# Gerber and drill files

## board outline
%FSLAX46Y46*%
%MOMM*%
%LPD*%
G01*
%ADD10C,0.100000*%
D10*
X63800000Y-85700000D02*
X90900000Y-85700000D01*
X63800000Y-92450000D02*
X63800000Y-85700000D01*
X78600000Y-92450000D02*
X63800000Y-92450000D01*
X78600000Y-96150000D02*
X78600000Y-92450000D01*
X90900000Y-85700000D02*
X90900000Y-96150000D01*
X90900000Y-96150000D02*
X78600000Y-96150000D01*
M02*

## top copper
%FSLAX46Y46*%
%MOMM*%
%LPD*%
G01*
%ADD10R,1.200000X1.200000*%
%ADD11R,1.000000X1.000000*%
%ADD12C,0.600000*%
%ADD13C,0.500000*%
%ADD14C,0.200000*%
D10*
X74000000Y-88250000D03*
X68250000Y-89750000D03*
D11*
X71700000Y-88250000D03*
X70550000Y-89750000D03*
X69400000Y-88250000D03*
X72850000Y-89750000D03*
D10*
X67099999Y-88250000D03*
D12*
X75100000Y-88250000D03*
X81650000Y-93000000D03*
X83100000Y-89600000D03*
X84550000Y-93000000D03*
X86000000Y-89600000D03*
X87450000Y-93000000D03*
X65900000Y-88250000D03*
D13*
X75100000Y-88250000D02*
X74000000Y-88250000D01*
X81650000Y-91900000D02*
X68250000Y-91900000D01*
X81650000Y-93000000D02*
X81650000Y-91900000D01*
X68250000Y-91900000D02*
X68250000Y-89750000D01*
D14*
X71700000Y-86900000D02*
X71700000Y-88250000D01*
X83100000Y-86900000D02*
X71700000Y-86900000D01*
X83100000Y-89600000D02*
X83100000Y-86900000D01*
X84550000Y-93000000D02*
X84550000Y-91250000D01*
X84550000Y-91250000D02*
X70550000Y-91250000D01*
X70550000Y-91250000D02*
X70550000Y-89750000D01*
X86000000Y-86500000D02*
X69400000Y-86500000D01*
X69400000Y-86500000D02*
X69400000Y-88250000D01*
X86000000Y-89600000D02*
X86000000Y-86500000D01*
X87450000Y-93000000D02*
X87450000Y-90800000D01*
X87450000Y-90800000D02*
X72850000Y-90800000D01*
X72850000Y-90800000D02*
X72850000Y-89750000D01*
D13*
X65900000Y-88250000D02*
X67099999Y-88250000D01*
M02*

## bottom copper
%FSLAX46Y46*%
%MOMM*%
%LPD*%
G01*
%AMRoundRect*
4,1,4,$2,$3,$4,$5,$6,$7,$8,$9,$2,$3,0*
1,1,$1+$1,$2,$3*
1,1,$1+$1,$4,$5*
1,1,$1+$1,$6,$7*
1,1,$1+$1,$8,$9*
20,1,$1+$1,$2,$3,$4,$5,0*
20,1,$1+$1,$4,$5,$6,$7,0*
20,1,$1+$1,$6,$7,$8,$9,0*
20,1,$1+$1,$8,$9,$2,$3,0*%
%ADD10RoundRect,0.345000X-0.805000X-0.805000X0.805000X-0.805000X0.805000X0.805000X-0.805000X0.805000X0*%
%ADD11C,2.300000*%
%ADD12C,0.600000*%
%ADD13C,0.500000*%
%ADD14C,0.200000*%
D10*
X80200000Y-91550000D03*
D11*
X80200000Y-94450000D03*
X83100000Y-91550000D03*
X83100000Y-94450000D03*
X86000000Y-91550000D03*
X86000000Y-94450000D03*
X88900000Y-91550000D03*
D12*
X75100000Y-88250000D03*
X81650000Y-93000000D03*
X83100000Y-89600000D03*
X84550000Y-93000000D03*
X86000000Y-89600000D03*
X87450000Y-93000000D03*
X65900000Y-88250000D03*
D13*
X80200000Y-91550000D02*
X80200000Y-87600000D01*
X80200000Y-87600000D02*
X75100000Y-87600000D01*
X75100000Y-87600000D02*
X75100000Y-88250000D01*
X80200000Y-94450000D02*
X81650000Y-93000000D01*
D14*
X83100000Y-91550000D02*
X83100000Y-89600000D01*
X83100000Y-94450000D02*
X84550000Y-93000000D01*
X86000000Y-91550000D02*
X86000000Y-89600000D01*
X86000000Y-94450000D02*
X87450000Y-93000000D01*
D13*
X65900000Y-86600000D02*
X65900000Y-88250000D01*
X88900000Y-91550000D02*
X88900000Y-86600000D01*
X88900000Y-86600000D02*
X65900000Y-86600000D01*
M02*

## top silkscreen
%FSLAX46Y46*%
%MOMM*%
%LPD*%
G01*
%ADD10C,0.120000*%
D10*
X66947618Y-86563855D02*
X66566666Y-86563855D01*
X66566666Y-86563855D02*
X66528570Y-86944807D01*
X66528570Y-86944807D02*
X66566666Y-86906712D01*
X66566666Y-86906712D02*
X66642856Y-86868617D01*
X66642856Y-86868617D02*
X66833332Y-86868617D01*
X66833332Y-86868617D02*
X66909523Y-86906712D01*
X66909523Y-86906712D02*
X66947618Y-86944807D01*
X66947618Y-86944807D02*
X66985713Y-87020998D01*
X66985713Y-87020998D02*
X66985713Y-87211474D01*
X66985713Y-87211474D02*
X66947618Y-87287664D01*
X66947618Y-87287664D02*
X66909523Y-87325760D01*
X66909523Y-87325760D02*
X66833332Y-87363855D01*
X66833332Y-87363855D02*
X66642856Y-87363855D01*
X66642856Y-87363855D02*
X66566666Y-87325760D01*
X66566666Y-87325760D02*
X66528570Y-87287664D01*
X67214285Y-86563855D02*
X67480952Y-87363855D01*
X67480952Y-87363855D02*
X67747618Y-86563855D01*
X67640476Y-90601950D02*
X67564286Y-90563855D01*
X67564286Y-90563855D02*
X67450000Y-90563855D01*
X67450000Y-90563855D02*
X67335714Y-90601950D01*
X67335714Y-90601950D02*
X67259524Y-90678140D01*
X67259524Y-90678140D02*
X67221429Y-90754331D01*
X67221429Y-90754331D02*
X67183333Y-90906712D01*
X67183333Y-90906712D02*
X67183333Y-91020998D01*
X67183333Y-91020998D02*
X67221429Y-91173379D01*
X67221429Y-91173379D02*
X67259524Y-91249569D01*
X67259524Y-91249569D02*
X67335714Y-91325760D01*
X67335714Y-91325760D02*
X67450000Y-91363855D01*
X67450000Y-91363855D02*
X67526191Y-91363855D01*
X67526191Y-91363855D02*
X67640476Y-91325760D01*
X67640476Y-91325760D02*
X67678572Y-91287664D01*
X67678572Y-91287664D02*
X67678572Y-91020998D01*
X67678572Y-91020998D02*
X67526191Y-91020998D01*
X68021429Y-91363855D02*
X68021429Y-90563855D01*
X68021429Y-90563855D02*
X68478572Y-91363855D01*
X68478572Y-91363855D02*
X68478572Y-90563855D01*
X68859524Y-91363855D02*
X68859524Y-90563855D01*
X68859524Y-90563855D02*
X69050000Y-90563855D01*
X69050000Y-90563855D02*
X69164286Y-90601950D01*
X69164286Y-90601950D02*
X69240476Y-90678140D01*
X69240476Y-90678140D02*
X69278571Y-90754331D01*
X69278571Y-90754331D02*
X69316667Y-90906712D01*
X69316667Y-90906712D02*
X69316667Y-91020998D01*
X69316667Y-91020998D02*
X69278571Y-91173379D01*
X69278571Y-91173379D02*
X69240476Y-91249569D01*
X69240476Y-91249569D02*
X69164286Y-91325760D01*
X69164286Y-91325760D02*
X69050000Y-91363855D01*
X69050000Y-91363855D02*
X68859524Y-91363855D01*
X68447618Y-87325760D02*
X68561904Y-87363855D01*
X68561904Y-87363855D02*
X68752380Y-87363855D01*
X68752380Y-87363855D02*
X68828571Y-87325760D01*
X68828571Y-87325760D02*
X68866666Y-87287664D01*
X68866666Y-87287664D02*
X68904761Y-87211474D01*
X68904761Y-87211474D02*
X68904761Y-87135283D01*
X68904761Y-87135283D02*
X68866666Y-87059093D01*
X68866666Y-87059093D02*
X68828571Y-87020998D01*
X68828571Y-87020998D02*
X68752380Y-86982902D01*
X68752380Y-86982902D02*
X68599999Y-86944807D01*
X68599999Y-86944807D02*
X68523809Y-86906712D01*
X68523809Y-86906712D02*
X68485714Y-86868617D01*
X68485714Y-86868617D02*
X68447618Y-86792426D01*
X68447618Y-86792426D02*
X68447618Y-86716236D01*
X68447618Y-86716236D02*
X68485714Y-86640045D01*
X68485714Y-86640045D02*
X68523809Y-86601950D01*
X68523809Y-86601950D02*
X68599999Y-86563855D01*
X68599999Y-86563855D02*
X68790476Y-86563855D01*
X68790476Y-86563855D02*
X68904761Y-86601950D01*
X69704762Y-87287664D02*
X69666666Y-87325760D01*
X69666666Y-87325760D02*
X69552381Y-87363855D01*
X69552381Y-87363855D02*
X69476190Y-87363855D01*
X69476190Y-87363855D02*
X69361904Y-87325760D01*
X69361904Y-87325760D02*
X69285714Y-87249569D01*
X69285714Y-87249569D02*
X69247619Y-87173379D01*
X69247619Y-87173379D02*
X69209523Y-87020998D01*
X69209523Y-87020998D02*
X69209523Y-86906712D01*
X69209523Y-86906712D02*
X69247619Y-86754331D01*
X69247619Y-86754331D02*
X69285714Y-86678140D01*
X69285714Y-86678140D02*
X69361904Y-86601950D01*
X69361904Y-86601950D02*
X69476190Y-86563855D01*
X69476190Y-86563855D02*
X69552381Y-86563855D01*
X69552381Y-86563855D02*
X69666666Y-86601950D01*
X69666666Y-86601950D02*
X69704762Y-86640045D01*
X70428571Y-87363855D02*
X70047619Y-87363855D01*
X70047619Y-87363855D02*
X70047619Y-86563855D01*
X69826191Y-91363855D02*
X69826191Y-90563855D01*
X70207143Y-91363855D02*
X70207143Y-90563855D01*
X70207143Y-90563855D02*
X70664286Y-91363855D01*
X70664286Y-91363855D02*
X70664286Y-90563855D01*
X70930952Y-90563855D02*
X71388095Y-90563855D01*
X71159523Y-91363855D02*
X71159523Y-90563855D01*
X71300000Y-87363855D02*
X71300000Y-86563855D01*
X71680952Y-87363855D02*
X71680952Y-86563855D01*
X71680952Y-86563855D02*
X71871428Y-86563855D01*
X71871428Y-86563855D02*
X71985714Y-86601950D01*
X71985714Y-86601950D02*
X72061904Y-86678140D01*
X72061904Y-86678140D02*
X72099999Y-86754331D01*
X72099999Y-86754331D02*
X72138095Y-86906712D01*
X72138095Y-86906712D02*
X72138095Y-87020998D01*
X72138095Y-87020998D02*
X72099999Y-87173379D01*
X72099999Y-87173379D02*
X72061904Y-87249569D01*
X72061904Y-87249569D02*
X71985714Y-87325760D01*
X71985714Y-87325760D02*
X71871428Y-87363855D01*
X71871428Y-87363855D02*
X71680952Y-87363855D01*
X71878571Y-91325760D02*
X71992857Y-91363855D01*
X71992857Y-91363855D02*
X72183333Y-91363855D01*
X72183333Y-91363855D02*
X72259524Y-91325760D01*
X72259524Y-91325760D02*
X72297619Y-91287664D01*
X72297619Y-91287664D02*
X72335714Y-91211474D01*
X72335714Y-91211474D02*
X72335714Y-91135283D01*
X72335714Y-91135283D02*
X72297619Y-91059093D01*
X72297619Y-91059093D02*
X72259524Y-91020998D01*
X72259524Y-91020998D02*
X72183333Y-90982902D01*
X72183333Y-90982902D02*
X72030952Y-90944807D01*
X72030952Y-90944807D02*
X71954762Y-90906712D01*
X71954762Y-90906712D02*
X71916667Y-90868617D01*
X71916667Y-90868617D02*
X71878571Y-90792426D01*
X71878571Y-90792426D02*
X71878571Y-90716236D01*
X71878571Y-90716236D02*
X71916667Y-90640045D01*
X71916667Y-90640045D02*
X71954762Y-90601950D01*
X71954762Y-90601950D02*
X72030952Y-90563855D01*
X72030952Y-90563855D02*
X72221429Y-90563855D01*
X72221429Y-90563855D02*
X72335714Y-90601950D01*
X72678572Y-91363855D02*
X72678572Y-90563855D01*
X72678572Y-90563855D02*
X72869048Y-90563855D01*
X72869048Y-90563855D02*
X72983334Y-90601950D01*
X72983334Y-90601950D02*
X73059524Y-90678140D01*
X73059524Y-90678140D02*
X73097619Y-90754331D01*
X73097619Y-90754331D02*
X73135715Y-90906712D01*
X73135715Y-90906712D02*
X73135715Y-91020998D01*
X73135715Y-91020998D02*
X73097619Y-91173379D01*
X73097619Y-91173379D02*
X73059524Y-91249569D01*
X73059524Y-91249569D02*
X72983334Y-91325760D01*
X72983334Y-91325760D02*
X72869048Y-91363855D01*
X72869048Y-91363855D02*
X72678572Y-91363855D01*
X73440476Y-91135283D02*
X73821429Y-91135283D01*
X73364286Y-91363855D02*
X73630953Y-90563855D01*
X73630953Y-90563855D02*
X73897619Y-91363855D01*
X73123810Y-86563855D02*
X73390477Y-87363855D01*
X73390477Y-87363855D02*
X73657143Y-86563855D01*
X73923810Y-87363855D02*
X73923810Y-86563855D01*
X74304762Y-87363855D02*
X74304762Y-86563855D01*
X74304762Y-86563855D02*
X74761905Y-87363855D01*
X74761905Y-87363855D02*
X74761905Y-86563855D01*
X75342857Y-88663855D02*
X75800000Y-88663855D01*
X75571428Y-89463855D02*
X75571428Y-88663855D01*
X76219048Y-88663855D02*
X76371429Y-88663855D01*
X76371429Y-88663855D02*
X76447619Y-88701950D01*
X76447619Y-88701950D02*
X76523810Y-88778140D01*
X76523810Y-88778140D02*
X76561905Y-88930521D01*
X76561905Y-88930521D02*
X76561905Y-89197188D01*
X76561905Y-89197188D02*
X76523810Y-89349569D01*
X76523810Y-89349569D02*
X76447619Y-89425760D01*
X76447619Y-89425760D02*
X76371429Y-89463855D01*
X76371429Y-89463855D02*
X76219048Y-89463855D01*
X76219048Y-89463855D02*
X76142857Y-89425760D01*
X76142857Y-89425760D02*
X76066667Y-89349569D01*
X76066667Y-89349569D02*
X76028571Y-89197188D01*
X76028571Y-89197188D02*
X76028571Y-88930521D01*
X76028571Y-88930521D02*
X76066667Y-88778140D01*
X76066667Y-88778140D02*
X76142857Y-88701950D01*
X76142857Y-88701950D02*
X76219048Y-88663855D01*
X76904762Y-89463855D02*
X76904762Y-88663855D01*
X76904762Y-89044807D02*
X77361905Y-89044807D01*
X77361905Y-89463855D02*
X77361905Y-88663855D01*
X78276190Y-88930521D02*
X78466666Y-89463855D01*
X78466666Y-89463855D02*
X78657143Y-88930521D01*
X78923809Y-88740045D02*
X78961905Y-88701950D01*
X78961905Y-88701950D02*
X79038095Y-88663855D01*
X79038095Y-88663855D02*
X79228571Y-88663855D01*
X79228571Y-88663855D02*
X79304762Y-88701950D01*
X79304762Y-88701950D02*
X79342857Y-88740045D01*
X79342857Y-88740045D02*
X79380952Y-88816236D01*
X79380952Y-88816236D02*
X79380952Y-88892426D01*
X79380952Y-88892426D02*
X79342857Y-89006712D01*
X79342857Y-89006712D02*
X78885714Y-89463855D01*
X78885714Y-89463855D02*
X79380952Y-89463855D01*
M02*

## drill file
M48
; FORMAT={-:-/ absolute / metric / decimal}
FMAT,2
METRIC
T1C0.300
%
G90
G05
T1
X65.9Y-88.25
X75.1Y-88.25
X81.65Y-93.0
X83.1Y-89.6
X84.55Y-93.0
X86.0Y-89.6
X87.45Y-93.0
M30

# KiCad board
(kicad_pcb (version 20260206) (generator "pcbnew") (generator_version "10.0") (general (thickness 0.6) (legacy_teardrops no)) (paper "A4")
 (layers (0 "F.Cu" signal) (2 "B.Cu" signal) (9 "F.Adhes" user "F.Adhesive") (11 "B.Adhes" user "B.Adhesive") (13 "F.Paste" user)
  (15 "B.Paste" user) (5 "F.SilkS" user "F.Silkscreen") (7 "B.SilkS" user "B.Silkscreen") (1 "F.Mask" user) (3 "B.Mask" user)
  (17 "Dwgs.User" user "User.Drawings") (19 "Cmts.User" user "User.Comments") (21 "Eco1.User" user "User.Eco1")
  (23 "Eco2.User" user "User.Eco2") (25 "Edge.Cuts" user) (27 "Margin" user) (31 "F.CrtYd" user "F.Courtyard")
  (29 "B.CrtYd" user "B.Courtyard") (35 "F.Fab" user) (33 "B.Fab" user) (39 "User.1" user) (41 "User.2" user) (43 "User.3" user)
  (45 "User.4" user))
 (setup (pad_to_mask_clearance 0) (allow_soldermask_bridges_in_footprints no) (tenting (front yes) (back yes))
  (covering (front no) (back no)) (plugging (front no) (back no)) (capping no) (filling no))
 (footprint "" (layer "F.Cu") (at 70.55 89)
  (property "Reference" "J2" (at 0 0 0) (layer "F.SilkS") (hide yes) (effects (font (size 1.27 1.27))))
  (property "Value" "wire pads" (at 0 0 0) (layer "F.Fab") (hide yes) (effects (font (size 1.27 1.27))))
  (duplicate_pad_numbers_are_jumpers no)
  (pad "1" smd rect (at 3.45 -0.75) (size 1.2 1.2) (layers "F.Cu" "F.Mask") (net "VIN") (thermal_bridge_angle 45))
  (pad "2" smd rect (at -2.3 0.75) (size 1.2 1.2) (layers "F.Cu" "F.Mask") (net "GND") (thermal_bridge_angle 45))
  (pad "3" smd rect (at 1.15 -0.75) (size 1 1) (layers "F.Cu" "F.Mask") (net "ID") (thermal_bridge_angle 45))
  (pad "4" smd rect (at 0 0.75) (size 1 1) (layers "F.Cu" "F.Mask") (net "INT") (thermal_bridge_angle 45))
  (pad "5" smd rect (at -1.15 -0.75) (size 1 1) (layers "F.Cu" "F.Mask") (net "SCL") (thermal_bridge_angle 45))
  (pad "6" smd rect (at 2.3 0.75) (size 1 1) (layers "F.Cu" "F.Mask") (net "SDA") (thermal_bridge_angle 45))
  (pad "7" smd rect (at -3.450001 -0.75) (size 1.2 1.2) (layers "F.Cu" "F.Mask") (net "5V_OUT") (thermal_bridge_angle 45)))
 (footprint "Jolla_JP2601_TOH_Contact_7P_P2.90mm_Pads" (layer "F.Cu") (at 80.2 91.55)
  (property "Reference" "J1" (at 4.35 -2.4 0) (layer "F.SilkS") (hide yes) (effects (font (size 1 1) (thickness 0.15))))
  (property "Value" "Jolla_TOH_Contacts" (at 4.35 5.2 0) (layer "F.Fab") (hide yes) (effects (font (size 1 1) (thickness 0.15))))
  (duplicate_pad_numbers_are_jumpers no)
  (pad "1" smd roundrect (at 0 0) (size 2.3 2.3) (layers "B.Cu" "B.Mask") (roundrect_rratio 0.15) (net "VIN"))
  (pad "2" smd circle (at 0 2.9) (size 2.3 2.3) (layers "B.Cu" "B.Mask") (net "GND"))
  (pad "3" smd circle (at 2.9 0) (size 2.3 2.3) (layers "B.Cu" "B.Mask") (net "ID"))
  (pad "4" smd circle (at 2.9 2.9) (size 2.3 2.3) (layers "B.Cu" "B.Mask") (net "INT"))
  (pad "5" smd circle (at 5.8 0) (size 2.3 2.3) (layers "B.Cu" "B.Mask") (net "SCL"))
  (pad "6" smd circle (at 5.8 2.9) (size 2.3 2.3) (layers "B.Cu" "B.Mask") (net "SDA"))
  (pad "7" smd circle (at 8.7 0) (size 2.3 2.3) (layers "B.Cu" "B.Mask") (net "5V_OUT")))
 (gr_line (start 63.8 85.7) (end 90.9 85.7) (stroke (width 0.1) (type default)) (layer "Edge.Cuts"))
 (gr_line (start 63.8 92.45) (end 63.8 85.7) (stroke (width 0.1) (type default)) (layer "Edge.Cuts"))
 (gr_line (start 78.6 92.45) (end 63.8 92.45) (stroke (width 0.1) (type default)) (layer "Edge.Cuts"))
 (gr_line (start 78.6 96.15) (end 78.6 92.45) (stroke (width 0.1) (type default)) (layer "Edge.Cuts"))
 (gr_line (start 90.9 85.7) (end 90.9 96.15) (stroke (width 0.1) (type default)) (layer "Edge.Cuts"))
 (gr_line (start 90.9 96.15) (end 78.6 96.15) (stroke (width 0.1) (type default)) (layer "Edge.Cuts"))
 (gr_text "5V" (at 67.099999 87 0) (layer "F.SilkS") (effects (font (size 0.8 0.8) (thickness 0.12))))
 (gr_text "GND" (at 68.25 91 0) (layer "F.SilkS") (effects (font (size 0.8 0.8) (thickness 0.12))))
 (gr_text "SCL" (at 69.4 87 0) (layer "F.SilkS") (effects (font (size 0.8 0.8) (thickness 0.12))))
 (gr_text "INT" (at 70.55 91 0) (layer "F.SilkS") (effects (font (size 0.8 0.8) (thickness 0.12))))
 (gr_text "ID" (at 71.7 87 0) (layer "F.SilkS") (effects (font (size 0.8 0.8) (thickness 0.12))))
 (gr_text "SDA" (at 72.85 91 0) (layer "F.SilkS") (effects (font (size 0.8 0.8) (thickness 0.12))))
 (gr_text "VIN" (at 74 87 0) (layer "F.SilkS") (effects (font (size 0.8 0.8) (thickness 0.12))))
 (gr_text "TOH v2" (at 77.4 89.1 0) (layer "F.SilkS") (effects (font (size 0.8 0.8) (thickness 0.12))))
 (segment (start 75.1 88.25) (end 74 88.25) (width 0.5) (layer "F.Cu") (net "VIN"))
 (via (at 75.1 88.25) (size 0.6) (drill 0.3) (layers "F.Cu" "B.Cu") (tenting (front yes) (back yes)) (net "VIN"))
 (segment (start 80.2 91.55) (end 80.2 87.6) (width 0.5) (layer "B.Cu") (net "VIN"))
 (segment (start 80.2 87.6) (end 75.1 87.6) (width 0.5) (layer "B.Cu") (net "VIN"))
 (segment (start 75.1 87.6) (end 75.1 88.25) (width 0.5) (layer "B.Cu") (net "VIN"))
 (segment (start 81.65 91.9) (end 68.25 91.9) (width 0.5) (layer "F.Cu") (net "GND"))
 (segment (start 81.65 93) (end 81.65 91.9) (width 0.5) (layer "F.Cu") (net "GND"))
 (segment (start 68.25 91.9) (end 68.25 89.75) (width 0.5) (layer "F.Cu") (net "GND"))
 (via (at 81.65 93) (size 0.6) (drill 0.3) (layers "F.Cu" "B.Cu") (tenting (front yes) (back yes)) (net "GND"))
 (segment (start 80.2 94.45) (end 81.65 93) (width 0.5) (layer "B.Cu") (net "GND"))
 (segment (start 71.7 86.9) (end 71.7 88.25) (width 0.2) (layer "F.Cu") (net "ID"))
 (segment (start 83.1 86.9) (end 71.7 86.9) (width 0.2) (layer "F.Cu") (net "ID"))
 (segment (start 83.1 89.6) (end 83.1 86.9) (width 0.2) (layer "F.Cu") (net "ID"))
 (via (at 83.1 89.6) (size 0.6) (drill 0.3) (layers "F.Cu" "B.Cu") (tenting (front yes) (back yes)) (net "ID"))
 (segment (start 83.1 91.55) (end 83.1 89.6) (width 0.2) (layer "B.Cu") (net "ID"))
 (segment (start 84.55 93) (end 84.55 91.25) (width 0.2) (layer "F.Cu") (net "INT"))
 (segment (start 84.55 91.25) (end 70.55 91.25) (width 0.2) (layer "F.Cu") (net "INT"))
 (segment (start 70.55 91.25) (end 70.55 89.75) (width 0.2) (layer "F.Cu") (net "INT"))
 (via (at 84.55 93) (size 0.6) (drill 0.3) (layers "F.Cu" "B.Cu") (tenting (front yes) (back yes)) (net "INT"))
 (segment (start 83.1 94.45) (end 84.55 93) (width 0.2) (layer "B.Cu") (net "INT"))
 (segment (start 86 86.5) (end 69.4 86.5) (width 0.2) (layer "F.Cu") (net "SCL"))
 (segment (start 69.4 86.5) (end 69.4 88.25) (width 0.2) (layer "F.Cu") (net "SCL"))
 (segment (start 86 89.6) (end 86 86.5) (width 0.2) (layer "F.Cu") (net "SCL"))
 (via (at 86 89.6) (size 0.6) (drill 0.3) (layers "F.Cu" "B.Cu") (tenting (front yes) (back yes)) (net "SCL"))
 (segment (start 86 91.55) (end 86 89.6) (width 0.2) (layer "B.Cu") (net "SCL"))
 (segment (start 87.45 93) (end 87.45 90.8) (width 0.2) (layer "F.Cu") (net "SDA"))
 (segment (start 87.45 90.8) (end 72.85 90.8) (width 0.2) (layer "F.Cu") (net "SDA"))
 (segment (start 72.85 90.8) (end 72.85 89.75) (width 0.2) (layer "F.Cu") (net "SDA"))
 (via (at 87.45 93) (size 0.6) (drill 0.3) (layers "F.Cu" "B.Cu") (tenting (front yes) (back yes)) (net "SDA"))
 (segment (start 86 94.45) (end 87.45 93) (width 0.2) (layer "B.Cu") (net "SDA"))
 (segment (start 65.9 88.25) (end 67.099999 88.25) (width 0.5) (layer "F.Cu") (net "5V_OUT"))
 (via (at 65.9 88.25) (size 0.6) (drill 0.3) (layers "F.Cu" "B.Cu") (tenting (front yes) (back yes)) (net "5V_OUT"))
 (segment (start 65.9 86.6) (end 65.9 88.25) (width 0.5) (layer "B.Cu") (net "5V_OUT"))
 (segment (start 88.9 91.55) (end 88.9 86.6) (width 0.5) (layer "B.Cu") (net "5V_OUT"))
 (segment (start 88.9 86.6) (end 65.9 86.6) (width 0.5) (layer "B.Cu") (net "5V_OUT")))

